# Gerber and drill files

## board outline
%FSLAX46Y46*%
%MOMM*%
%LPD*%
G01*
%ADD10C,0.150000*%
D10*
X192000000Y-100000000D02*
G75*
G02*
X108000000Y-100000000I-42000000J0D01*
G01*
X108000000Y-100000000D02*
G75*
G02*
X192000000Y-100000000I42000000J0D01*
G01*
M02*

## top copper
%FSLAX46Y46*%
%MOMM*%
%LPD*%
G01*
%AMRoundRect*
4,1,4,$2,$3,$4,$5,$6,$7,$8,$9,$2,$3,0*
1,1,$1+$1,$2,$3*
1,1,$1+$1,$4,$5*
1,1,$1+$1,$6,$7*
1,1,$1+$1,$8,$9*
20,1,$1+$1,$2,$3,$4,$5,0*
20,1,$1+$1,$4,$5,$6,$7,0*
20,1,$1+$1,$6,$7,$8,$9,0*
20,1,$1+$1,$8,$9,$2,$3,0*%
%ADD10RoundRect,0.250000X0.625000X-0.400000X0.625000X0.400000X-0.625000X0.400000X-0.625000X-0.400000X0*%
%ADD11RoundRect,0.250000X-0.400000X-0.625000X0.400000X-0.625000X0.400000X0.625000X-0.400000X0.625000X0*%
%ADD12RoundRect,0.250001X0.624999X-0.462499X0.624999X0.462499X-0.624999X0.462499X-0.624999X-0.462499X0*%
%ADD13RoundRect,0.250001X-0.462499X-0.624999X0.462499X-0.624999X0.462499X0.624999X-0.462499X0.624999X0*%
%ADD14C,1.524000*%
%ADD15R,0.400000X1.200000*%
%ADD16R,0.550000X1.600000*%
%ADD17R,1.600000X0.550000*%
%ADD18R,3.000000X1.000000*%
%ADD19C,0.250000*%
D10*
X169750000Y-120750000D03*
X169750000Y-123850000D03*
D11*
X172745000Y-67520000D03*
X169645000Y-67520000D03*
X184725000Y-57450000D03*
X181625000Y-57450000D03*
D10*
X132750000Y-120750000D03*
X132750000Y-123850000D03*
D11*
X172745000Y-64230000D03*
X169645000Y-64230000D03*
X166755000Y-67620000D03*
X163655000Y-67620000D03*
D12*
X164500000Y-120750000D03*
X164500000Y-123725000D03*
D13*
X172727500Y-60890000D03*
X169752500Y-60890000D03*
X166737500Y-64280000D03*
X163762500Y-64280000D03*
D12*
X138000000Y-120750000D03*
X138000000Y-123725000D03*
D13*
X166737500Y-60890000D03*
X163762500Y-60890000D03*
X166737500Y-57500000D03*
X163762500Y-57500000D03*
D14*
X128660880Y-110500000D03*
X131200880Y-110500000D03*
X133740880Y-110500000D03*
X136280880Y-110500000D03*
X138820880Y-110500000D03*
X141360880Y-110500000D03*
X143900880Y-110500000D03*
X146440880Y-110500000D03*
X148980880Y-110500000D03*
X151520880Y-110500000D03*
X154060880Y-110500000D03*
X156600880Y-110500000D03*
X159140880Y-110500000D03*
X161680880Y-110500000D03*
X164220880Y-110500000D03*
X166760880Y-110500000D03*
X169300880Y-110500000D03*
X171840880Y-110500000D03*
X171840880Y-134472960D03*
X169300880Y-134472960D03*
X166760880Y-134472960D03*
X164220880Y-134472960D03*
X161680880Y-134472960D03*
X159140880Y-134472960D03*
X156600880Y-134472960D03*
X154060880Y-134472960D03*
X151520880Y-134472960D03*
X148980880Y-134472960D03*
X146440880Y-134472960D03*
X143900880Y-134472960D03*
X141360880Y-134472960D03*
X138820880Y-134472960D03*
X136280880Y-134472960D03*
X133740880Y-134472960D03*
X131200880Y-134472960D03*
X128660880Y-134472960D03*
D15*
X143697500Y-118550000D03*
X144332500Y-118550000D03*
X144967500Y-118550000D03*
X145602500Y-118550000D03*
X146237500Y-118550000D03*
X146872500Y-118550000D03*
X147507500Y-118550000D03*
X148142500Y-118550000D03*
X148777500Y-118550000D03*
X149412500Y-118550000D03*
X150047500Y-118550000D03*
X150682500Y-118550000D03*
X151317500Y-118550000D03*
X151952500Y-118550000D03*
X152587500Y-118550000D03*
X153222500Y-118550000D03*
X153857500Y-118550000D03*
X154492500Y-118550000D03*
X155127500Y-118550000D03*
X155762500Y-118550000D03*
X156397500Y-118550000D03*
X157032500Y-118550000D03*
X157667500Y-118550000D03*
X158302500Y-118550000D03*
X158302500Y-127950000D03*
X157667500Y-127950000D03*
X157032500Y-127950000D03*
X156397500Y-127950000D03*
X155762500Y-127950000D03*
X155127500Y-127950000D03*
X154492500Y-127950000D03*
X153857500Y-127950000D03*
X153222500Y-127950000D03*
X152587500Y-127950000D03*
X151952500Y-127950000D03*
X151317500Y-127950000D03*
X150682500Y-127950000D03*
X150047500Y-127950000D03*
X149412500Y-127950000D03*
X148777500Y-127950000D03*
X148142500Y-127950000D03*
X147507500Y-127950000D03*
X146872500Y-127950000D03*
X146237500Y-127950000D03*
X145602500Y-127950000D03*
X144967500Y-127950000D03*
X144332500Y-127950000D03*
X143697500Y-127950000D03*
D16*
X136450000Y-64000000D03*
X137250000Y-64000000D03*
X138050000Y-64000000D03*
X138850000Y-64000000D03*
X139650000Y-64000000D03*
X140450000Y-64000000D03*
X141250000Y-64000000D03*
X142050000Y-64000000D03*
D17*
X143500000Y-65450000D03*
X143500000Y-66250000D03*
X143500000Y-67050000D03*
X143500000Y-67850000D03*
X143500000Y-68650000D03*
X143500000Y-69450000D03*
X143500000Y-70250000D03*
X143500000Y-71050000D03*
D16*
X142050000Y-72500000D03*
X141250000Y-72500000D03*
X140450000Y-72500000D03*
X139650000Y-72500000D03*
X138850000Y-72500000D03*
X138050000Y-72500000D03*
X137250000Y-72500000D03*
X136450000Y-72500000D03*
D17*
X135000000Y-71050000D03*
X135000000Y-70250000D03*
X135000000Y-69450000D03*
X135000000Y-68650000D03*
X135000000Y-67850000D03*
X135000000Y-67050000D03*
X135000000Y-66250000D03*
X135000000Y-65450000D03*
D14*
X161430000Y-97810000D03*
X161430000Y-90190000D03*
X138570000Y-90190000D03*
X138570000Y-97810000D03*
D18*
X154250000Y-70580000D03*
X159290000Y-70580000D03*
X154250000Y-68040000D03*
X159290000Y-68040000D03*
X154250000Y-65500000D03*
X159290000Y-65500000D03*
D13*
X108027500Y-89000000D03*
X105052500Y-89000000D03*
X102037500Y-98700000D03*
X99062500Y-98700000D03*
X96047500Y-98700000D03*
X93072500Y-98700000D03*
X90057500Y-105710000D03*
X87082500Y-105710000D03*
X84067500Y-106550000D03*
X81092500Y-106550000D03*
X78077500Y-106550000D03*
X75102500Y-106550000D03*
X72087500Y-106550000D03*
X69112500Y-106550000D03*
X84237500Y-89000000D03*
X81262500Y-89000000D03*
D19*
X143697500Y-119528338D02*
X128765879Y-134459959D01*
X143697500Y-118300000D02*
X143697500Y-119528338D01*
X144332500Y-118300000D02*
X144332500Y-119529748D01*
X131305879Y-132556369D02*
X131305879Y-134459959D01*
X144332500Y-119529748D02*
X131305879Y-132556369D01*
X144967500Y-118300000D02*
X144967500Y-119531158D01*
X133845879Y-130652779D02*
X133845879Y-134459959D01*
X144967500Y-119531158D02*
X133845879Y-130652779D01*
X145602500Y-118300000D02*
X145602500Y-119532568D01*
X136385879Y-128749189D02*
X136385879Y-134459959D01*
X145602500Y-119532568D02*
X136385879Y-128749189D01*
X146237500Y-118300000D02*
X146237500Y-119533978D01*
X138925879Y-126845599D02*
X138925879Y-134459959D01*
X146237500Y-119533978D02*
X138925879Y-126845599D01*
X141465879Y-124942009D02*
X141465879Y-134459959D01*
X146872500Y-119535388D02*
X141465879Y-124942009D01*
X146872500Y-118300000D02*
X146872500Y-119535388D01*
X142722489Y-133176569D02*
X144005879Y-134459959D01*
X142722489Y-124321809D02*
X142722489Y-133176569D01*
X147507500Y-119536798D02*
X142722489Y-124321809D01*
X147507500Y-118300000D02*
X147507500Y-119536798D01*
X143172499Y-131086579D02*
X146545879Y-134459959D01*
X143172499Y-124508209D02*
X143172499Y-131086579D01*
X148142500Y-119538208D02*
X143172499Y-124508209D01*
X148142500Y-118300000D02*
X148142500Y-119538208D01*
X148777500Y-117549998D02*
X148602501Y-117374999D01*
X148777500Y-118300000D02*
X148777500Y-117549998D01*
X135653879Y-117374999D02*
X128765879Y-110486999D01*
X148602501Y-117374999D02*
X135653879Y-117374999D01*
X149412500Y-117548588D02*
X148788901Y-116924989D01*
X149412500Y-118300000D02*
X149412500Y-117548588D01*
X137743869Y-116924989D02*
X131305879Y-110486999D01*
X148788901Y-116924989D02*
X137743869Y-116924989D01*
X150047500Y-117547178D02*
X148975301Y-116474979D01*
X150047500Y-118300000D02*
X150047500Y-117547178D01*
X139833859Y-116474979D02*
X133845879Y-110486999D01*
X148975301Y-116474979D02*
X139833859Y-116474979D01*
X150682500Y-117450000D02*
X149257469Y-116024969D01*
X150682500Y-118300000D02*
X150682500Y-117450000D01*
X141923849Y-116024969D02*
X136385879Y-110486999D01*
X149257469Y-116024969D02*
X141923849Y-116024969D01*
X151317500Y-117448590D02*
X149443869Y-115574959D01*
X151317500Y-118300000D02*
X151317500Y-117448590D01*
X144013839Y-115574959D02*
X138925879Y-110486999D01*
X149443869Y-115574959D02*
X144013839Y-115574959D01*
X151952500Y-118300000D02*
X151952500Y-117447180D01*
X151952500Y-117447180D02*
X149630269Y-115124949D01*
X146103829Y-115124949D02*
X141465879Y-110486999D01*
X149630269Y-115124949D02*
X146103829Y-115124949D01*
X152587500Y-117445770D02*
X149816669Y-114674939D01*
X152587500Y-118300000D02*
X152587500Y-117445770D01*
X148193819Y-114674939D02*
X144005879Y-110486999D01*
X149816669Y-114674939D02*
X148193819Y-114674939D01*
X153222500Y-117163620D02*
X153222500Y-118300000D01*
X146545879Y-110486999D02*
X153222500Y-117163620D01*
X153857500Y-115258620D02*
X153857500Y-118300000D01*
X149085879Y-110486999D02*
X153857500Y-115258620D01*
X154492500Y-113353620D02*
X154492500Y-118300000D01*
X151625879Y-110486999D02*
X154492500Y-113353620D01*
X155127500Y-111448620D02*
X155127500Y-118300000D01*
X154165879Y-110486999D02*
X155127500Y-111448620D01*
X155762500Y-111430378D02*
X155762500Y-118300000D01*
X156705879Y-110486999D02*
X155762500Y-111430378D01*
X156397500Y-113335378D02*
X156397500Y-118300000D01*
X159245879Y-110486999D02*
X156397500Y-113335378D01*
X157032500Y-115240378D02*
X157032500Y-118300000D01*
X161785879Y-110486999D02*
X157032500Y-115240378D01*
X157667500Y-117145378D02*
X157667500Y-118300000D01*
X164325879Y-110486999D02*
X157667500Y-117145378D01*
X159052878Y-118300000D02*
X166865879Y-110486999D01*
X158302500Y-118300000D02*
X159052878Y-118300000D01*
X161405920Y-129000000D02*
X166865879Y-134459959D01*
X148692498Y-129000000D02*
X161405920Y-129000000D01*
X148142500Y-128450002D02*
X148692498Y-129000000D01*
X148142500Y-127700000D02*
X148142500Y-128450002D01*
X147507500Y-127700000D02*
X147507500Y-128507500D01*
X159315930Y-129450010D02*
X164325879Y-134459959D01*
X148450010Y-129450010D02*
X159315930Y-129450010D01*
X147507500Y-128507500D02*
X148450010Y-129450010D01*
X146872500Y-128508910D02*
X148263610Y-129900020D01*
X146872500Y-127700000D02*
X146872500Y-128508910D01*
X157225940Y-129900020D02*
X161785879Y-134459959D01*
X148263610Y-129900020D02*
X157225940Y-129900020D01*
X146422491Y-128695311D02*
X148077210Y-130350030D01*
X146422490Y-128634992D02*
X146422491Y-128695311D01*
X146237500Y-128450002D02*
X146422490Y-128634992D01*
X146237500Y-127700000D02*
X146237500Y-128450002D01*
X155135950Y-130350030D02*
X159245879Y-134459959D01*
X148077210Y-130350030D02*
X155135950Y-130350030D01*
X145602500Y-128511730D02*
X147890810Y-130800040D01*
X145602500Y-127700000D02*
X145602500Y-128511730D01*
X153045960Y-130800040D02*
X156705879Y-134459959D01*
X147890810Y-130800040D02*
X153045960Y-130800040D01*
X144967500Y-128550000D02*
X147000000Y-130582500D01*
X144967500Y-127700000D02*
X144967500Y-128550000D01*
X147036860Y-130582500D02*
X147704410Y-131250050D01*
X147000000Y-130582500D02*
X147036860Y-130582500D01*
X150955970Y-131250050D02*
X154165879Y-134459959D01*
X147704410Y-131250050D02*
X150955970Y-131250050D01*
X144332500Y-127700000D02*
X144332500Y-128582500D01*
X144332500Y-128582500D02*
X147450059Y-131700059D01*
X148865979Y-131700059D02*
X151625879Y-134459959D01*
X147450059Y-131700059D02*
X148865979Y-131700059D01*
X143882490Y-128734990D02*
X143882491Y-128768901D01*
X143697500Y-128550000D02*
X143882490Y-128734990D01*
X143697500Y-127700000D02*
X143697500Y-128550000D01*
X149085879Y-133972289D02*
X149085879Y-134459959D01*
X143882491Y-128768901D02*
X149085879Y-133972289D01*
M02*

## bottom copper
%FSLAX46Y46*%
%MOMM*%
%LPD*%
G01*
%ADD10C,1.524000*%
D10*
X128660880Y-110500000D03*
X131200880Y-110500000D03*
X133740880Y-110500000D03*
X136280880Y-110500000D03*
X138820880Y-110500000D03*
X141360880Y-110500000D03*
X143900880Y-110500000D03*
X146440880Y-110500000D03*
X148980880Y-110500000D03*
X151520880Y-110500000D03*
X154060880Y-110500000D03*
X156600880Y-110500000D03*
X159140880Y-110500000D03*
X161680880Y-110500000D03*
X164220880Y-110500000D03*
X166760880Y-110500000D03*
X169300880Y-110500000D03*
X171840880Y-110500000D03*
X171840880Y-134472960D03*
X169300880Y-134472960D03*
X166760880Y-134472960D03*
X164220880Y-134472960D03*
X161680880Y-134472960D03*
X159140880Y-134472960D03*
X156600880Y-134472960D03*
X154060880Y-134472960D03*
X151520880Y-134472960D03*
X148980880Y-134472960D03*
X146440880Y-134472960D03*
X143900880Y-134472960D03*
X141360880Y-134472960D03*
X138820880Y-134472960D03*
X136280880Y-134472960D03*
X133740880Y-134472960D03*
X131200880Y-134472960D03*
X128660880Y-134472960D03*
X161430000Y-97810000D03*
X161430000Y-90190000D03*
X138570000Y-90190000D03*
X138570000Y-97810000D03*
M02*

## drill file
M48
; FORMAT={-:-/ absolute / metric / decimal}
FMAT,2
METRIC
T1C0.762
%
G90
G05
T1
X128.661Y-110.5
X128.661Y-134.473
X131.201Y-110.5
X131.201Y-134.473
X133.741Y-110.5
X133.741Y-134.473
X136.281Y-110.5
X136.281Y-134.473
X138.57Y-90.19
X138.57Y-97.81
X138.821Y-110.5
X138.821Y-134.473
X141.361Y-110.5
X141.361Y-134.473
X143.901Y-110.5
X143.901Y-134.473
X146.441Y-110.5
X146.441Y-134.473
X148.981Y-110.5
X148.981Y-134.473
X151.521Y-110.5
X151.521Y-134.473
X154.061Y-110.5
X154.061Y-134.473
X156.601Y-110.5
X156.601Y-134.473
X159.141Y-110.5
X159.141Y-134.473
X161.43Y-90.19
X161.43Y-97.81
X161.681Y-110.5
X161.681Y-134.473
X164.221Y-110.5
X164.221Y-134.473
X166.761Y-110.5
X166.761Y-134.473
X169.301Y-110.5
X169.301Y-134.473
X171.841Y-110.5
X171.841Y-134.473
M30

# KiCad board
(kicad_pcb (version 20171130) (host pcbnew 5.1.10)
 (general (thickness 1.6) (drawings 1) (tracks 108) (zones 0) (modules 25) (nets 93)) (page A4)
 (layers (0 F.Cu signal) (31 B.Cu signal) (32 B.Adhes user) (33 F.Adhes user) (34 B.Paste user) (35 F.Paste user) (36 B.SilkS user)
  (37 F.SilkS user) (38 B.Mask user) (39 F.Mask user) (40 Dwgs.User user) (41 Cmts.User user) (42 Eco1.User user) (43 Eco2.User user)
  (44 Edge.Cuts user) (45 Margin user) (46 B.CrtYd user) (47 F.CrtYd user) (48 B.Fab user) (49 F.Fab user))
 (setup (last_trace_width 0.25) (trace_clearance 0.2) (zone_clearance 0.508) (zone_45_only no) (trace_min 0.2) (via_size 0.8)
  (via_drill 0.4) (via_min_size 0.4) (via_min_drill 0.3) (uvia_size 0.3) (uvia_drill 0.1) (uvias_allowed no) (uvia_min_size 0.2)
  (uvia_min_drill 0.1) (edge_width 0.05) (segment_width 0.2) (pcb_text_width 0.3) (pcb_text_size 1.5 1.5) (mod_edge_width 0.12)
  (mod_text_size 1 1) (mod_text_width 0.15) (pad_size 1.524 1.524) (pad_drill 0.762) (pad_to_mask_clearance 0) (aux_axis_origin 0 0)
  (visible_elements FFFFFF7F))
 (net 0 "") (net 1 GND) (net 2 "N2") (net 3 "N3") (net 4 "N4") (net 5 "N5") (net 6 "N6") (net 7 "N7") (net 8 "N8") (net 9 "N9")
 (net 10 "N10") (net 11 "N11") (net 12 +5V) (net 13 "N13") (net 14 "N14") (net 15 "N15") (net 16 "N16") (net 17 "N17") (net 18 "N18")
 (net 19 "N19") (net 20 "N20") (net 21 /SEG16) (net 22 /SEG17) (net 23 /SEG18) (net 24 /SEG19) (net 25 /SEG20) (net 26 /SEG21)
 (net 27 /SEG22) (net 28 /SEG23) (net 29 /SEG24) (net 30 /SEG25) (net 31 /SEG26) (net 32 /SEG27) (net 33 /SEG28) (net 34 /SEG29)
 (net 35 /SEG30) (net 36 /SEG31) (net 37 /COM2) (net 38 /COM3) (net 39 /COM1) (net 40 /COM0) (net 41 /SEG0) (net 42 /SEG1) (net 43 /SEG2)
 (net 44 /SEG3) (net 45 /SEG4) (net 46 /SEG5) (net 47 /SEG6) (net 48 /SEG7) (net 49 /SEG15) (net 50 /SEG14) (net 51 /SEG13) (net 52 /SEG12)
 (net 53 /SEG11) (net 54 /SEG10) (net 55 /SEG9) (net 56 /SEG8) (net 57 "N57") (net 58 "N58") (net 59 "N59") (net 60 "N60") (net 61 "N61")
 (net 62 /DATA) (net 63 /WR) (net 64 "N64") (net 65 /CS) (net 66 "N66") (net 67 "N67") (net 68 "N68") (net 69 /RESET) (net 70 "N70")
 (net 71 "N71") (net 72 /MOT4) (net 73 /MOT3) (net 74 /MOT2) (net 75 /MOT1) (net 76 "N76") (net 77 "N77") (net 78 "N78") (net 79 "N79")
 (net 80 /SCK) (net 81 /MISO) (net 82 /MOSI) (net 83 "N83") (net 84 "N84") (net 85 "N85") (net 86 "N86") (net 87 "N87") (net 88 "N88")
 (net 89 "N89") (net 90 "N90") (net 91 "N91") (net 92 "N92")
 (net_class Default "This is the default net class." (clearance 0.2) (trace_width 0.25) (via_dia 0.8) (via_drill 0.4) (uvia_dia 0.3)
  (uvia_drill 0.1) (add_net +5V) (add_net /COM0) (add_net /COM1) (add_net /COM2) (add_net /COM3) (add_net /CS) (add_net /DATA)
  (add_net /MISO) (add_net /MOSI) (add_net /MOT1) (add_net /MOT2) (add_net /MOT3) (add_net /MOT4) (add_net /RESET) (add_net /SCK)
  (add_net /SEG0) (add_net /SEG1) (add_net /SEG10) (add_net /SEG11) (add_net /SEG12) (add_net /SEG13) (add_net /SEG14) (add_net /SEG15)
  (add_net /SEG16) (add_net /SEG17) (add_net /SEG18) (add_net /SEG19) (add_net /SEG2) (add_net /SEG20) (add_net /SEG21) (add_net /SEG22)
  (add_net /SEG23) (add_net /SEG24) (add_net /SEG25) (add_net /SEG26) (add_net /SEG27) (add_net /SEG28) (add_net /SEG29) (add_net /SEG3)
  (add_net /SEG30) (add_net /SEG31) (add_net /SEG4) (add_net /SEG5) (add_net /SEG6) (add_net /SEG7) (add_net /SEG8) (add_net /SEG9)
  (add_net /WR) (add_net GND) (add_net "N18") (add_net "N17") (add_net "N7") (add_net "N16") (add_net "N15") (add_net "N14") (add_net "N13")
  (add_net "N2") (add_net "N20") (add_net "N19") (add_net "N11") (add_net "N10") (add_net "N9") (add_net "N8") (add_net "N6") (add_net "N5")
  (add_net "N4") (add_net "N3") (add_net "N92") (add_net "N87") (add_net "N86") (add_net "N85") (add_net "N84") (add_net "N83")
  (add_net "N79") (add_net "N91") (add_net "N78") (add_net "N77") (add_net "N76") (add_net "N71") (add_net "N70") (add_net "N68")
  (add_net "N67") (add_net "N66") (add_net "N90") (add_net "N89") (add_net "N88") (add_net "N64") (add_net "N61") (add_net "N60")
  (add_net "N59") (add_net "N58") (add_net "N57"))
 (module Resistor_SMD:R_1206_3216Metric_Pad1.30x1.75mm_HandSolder (layer F.Cu) (at 169.75 122.3 90)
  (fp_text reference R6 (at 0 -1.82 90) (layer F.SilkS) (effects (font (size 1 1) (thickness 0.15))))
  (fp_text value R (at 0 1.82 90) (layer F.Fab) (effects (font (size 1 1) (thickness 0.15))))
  (pad 2 smd roundrect (at 1.55 0 90) (size 1.3 1.75) (layers F.Cu F.Paste F.Mask) (roundrect_rratio 0.192308) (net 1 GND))
  (pad 1 smd roundrect (at -1.55 0 90) (size 1.3 1.75) (layers F.Cu F.Paste F.Mask) (roundrect_rratio 0.192308) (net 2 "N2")))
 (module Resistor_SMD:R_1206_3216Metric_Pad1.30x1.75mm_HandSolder (layer F.Cu) (at 171.195 67.52)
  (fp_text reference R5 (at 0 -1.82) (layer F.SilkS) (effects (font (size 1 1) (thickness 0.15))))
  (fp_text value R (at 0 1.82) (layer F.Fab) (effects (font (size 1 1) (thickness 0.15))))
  (pad 2 smd roundrect (at 1.55 0) (size 1.3 1.75) (layers F.Cu F.Paste F.Mask) (roundrect_rratio 0.192308) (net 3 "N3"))
  (pad 1 smd roundrect (at -1.55 0) (size 1.3 1.75) (layers F.Cu F.Paste F.Mask) (roundrect_rratio 0.192308) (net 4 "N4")))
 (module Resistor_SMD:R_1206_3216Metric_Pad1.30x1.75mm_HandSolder (layer F.Cu) (at 183.175 57.45)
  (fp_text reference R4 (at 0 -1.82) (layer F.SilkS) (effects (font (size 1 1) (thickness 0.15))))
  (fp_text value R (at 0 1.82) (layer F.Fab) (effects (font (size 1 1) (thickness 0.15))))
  (pad 2 smd roundrect (at 1.55 0) (size 1.3 1.75) (layers F.Cu F.Paste F.Mask) (roundrect_rratio 0.192308) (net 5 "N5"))
  (pad 1 smd roundrect (at -1.55 0) (size 1.3 1.75) (layers F.Cu F.Paste F.Mask) (roundrect_rratio 0.192308) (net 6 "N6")))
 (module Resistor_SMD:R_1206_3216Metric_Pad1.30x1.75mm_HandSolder (layer F.Cu) (at 132.75 122.3 90)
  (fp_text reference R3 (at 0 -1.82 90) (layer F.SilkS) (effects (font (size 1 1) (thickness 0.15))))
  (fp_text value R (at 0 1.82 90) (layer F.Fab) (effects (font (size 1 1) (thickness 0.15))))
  (pad 2 smd roundrect (at 1.55 0 90) (size 1.3 1.75) (layers F.Cu F.Paste F.Mask) (roundrect_rratio 0.192308) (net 1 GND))
  (pad 1 smd roundrect (at -1.55 0 90) (size 1.3 1.75) (layers F.Cu F.Paste F.Mask) (roundrect_rratio 0.192308) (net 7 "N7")))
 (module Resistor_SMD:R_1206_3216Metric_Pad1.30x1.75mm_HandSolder (layer F.Cu) (at 171.195 64.23)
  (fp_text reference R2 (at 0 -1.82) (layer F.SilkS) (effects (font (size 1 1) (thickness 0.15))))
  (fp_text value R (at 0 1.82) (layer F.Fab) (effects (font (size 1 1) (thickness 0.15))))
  (pad 2 smd roundrect (at 1.55 0) (size 1.3 1.75) (layers F.Cu F.Paste F.Mask) (roundrect_rratio 0.192308) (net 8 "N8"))
  (pad 1 smd roundrect (at -1.55 0) (size 1.3 1.75) (layers F.Cu F.Paste F.Mask) (roundrect_rratio 0.192308) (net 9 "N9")))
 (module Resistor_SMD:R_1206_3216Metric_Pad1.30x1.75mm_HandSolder (layer F.Cu) (at 165.205 67.62)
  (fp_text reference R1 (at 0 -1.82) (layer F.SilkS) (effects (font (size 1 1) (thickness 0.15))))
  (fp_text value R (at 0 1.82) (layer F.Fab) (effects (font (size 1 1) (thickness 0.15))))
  (pad 2 smd roundrect (at 1.55 0) (size 1.3 1.75) (layers F.Cu F.Paste F.Mask) (roundrect_rratio 0.192308) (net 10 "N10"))
  (pad 1 smd roundrect (at -1.55 0) (size 1.3 1.75) (layers F.Cu F.Paste F.Mask) (roundrect_rratio 0.192308) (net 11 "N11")))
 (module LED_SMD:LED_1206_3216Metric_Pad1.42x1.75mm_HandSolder (layer F.Cu) (at 164.5 122.2375 90)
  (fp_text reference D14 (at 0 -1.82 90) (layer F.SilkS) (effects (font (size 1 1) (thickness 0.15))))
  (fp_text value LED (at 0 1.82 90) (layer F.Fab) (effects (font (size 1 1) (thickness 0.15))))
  (pad 2 smd roundrect (at 1.4875 0 90) (size 1.425 1.75) (layers F.Cu F.Paste F.Mask) (roundrect_rratio 0.175439) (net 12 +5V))
  (pad 1 smd roundrect (at -1.4875 0 90) (size 1.425 1.75) (layers F.Cu F.Paste F.Mask) (roundrect_rratio 0.175439) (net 2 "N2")))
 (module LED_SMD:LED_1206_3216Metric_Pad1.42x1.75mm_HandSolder (layer F.Cu) (at 171.24 60.89)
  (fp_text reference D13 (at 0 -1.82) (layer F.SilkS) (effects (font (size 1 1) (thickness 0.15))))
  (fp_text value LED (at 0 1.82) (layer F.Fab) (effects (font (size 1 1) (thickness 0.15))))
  (pad 2 smd roundrect (at 1.4875 0) (size 1.425 1.75) (layers F.Cu F.Paste F.Mask) (roundrect_rratio 0.175439) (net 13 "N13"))
  (pad 1 smd roundrect (at -1.4875 0) (size 1.425 1.75) (layers F.Cu F.Paste F.Mask) (roundrect_rratio 0.175439) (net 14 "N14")))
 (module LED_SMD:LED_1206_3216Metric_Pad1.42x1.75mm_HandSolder (layer F.Cu) (at 165.25 64.28)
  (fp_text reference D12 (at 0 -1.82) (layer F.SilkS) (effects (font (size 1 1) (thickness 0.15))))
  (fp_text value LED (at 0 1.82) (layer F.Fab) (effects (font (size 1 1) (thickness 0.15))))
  (pad 2 smd roundrect (at 1.4875 0) (size 1.425 1.75) (layers F.Cu F.Paste F.Mask) (roundrect_rratio 0.175439) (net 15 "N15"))
  (pad 1 smd roundrect (at -1.4875 0) (size 1.425 1.75) (layers F.Cu F.Paste F.Mask) (roundrect_rratio 0.175439) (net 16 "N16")))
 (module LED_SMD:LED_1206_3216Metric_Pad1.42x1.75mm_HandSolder (layer F.Cu) (at 138 122.2375 90)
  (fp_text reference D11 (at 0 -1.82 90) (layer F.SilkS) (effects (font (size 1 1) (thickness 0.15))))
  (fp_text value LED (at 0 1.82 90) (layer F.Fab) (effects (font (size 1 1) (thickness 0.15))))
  (pad 2 smd roundrect (at 1.4875 0 90) (size 1.425 1.75) (layers F.Cu F.Paste F.Mask) (roundrect_rratio 0.175439) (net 12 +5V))
  (pad 1 smd roundrect (at -1.4875 0 90) (size 1.425 1.75) (layers F.Cu F.Paste F.Mask) (roundrect_rratio 0.175439) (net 7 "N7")))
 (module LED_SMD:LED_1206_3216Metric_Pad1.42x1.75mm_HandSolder (layer F.Cu) (at 165.25 60.89)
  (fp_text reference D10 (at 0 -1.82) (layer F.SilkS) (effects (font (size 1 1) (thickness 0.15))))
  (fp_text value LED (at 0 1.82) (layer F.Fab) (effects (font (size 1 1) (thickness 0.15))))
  (pad 2 smd roundrect (at 1.4875 0) (size 1.425 1.75) (layers F.Cu F.Paste F.Mask) (roundrect_rratio 0.175439) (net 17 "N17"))
  (pad 1 smd roundrect (at -1.4875 0) (size 1.425 1.75) (layers F.Cu F.Paste F.Mask) (roundrect_rratio 0.175439) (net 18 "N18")))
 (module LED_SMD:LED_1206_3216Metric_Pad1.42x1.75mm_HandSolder (layer F.Cu) (at 165.25 57.5)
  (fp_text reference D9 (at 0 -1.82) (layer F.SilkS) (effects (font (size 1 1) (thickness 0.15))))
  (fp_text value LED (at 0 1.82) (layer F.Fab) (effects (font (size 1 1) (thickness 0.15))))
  (pad 2 smd roundrect (at 1.4875 0) (size 1.425 1.75) (layers F.Cu F.Paste F.Mask) (roundrect_rratio 0.175439) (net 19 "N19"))
  (pad 1 smd roundrect (at -1.4875 0) (size 1.425 1.75) (layers F.Cu F.Paste F.Mask) (roundrect_rratio 0.175439) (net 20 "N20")))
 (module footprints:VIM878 (layer F.Cu) (at 124.25 112.97296)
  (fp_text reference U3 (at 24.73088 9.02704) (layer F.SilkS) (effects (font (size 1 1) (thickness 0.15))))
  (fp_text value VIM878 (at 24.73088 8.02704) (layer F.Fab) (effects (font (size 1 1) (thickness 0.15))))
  (pad 36 thru_hole circle (at 4.41088 -2.47296) (size 1.524 1.524) (drill 0.762) (layers *.Cu *.Mask) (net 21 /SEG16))
  (pad 35 thru_hole circle (at 6.95088 -2.47296) (size 1.524 1.524) (drill 0.762) (layers *.Cu *.Mask) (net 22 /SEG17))
  (pad 34 thru_hole circle (at 9.49088 -2.47296) (size 1.524 1.524) (drill 0.762) (layers *.Cu *.Mask) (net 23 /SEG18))
  (pad 33 thru_hole circle (at 12.03088 -2.47296) (size 1.524 1.524) (drill 0.762) (layers *.Cu *.Mask) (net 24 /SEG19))
  (pad 32 thru_hole circle (at 14.57088 -2.47296) (size 1.524 1.524) (drill 0.762) (layers *.Cu *.Mask) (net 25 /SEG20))
  (pad 31 thru_hole circle (at 17.11088 -2.47296) (size 1.524 1.524) (drill 0.762) (layers *.Cu *.Mask) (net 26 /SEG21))
  (pad 30 thru_hole circle (at 19.65088 -2.47296) (size 1.524 1.524) (drill 0.762) (layers *.Cu *.Mask) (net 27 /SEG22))
  (pad 29 thru_hole circle (at 22.19088 -2.47296) (size 1.524 1.524) (drill 0.762) (layers *.Cu *.Mask) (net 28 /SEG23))
  (pad 28 thru_hole circle (at 24.73088 -2.47296) (size 1.524 1.524) (drill 0.762) (layers *.Cu *.Mask) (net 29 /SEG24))
  (pad 27 thru_hole circle (at 27.27088 -2.47296) (size 1.524 1.524) (drill 0.762) (layers *.Cu *.Mask) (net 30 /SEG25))
  (pad 26 thru_hole circle (at 29.81088 -2.47296) (size 1.524 1.524) (drill 0.762) (layers *.Cu *.Mask) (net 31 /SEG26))
  (pad 25 thru_hole circle (at 32.35088 -2.47296) (size 1.524 1.524) (drill 0.762) (layers *.Cu *.Mask) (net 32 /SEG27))
  (pad 24 thru_hole circle (at 34.89088 -2.47296) (size 1.524 1.524) (drill 0.762) (layers *.Cu *.Mask) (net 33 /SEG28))
  (pad 23 thru_hole circle (at 37.43088 -2.47296) (size 1.524 1.524) (drill 0.762) (layers *.Cu *.Mask) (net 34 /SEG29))
  (pad 22 thru_hole circle (at 39.97088 -2.47296) (size 1.524 1.524) (drill 0.762) (layers *.Cu *.Mask) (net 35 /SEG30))
  (pad 21 thru_hole circle (at 42.51088 -2.47296) (size 1.524 1.524) (drill 0.762) (layers *.Cu *.Mask) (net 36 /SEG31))
  (pad 20 thru_hole circle (at 45.05088 -2.47296) (size 1.524 1.524) (drill 0.762) (layers *.Cu *.Mask) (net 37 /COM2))
  (pad 19 thru_hole circle (at 47.59088 -2.47296) (size 1.524 1.524) (drill 0.762) (layers *.Cu *.Mask) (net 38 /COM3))
  (pad 18 thru_hole circle (at 47.59088 21.5) (size 1.524 1.524) (drill 0.762) (layers *.Cu *.Mask) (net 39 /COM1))
  (pad 17 thru_hole circle (at 45.05088 21.5) (size 1.524 1.524) (drill 0.762) (layers *.Cu *.Mask) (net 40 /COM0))
  (pad 16 thru_hole circle (at 42.51088 21.5) (size 1.524 1.524) (drill 0.762) (layers *.Cu *.Mask) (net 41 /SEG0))
  (pad 15 thru_hole circle (at 39.97088 21.5) (size 1.524 1.524) (drill 0.762) (layers *.Cu *.Mask) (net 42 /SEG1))
  (pad 14 thru_hole circle (at 37.43088 21.5) (size 1.524 1.524) (drill 0.762) (layers *.Cu *.Mask) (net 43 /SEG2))
  (pad 13 thru_hole circle (at 34.89088 21.5) (size 1.524 1.524) (drill 0.762) (layers *.Cu *.Mask) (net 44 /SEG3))
  (pad 12 thru_hole circle (at 32.35088 21.5) (size 1.524 1.524) (drill 0.762) (layers *.Cu *.Mask) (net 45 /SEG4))
  (pad 11 thru_hole circle (at 29.81088 21.5) (size 1.524 1.524) (drill 0.762) (layers *.Cu *.Mask) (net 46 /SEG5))
  (pad 10 thru_hole circle (at 27.27088 21.5) (size 1.524 1.524) (drill 0.762) (layers *.Cu *.Mask) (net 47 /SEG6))
  (pad 9 thru_hole circle (at 24.73088 21.5) (size 1.524 1.524) (drill 0.762) (layers *.Cu *.Mask) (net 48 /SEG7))
  (pad 8 thru_hole circle (at 22.19088 21.5) (size 1.524 1.524) (drill 0.762) (layers *.Cu *.Mask) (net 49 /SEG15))
  (pad 7 thru_hole circle (at 19.65088 21.5) (size 1.524 1.524) (drill 0.762) (layers *.Cu *.Mask) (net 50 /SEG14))
  (pad 6 thru_hole circle (at 17.11088 21.5) (size 1.524 1.524) (drill 0.762) (layers *.Cu *.Mask) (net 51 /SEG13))
  (pad 5 thru_hole circle (at 14.57088 21.5) (size 1.524 1.524) (drill 0.762) (layers *.Cu *.Mask) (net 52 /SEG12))
  (pad 4 thru_hole circle (at 12.03088 21.5) (size 1.524 1.524) (drill 0.762) (layers *.Cu *.Mask) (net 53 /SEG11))
  (pad 3 thru_hole circle (at 9.49088 21.5) (size 1.524 1.524) (drill 0.762) (layers *.Cu *.Mask) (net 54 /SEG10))
  (pad 2 thru_hole circle (at 6.95088 21.5) (size 1.524 1.524) (drill 0.762) (layers *.Cu *.Mask) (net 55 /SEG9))
  (pad 1 thru_hole circle (at 4.41088 21.5) (size 1.524 1.524) (drill 0.762) (layers *.Cu *.Mask) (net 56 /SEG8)))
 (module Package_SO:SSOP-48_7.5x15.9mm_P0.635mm (layer F.Cu) (at 151 123.25 90)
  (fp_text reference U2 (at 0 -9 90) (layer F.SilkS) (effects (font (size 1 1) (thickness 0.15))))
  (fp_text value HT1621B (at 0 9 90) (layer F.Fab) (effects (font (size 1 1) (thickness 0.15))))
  (pad 48 smd rect (at 4.7 -7.3025 90) (size 1.2 0.4) (layers F.Cu F.Paste F.Mask) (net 56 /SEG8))
  (pad 47 smd rect (at 4.7 -6.6675 90) (size 1.2 0.4) (layers F.Cu F.Paste F.Mask) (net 55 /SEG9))
  (pad 46 smd rect (at 4.7 -6.0325 90) (size 1.2 0.4) (layers F.Cu F.Paste F.Mask) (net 54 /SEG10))
  (pad 45 smd rect (at 4.7 -5.3975 90) (size 1.2 0.4) (layers F.Cu F.Paste F.Mask) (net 53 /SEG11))
  (pad 44 smd rect (at 4.7 -4.7625 90) (size 1.2 0.4) (layers F.Cu F.Paste F.Mask) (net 52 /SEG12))
  (pad 43 smd rect (at 4.7 -4.1275 90) (size 1.2 0.4) (layers F.Cu F.Paste F.Mask) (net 51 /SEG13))
  (pad 42 smd rect (at 4.7 -3.4925 90) (size 1.2 0.4) (layers F.Cu F.Paste F.Mask) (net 50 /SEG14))
  (pad 41 smd rect (at 4.7 -2.8575 90) (size 1.2 0.4) (layers F.Cu F.Paste F.Mask) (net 49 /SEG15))
  (pad 40 smd rect (at 4.7 -2.2225 90) (size 1.2 0.4) (layers F.Cu F.Paste F.Mask) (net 21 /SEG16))
  (pad 39 smd rect (at 4.7 -1.5875 90) (size 1.2 0.4) (layers F.Cu F.Paste F.Mask) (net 22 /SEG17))
  (pad 38 smd rect (at 4.7 -0.9525 90) (size 1.2 0.4) (layers F.Cu F.Paste F.Mask) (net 23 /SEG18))
  (pad 37 smd rect (at 4.7 -0.3175 90) (size 1.2 0.4) (layers F.Cu F.Paste F.Mask) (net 24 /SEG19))
  (pad 36 smd rect (at 4.7 0.3175 90) (size 1.2 0.4) (layers F.Cu F.Paste F.Mask) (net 25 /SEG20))
  (pad 35 smd rect (at 4.7 0.9525 90) (size 1.2 0.4) (layers F.Cu F.Paste F.Mask) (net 26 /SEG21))
  (pad 34 smd rect (at 4.7 1.5875 90) (size 1.2 0.4) (layers F.Cu F.Paste F.Mask) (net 27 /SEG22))
  (pad 33 smd rect (at 4.7 2.2225 90) (size 1.2 0.4) (layers F.Cu F.Paste F.Mask) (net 28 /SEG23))
  (pad 32 smd rect (at 4.7 2.8575 90) (size 1.2 0.4) (layers F.Cu F.Paste F.Mask) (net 29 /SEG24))
  (pad 31 smd rect (at 4.7 3.4925 90) (size 1.2 0.4) (layers F.Cu F.Paste F.Mask) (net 30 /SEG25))
  (pad 30 smd rect (at 4.7 4.1275 90) (size 1.2 0.4) (layers F.Cu F.Paste F.Mask) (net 31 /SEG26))
  (pad 29 smd rect (at 4.7 4.7625 90) (size 1.2 0.4) (layers F.Cu F.Paste F.Mask) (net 32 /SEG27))
  (pad 28 smd rect (at 4.7 5.3975 90) (size 1.2 0.4) (layers F.Cu F.Paste F.Mask) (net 33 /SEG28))
  (pad 27 smd rect (at 4.7 6.0325 90) (size 1.2 0.4) (layers F.Cu F.Paste F.Mask) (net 34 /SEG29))
  (pad 26 smd rect (at 4.7 6.6675 90) (size 1.2 0.4) (layers F.Cu F.Paste F.Mask) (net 35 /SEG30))
  (pad 25 smd rect (at 4.7 7.3025 90) (size 1.2 0.4) (layers F.Cu F.Paste F.Mask) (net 36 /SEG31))
  (pad 24 smd rect (at -4.7 7.3025 90) (size 1.2 0.4) (layers F.Cu F.Paste F.Mask) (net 38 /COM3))
  (pad 23 smd rect (at -4.7 6.6675 90) (size 1.2 0.4) (layers F.Cu F.Paste F.Mask) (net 37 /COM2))
  (pad 22 smd rect (at -4.7 6.0325 90) (size 1.2 0.4) (layers F.Cu F.Paste F.Mask) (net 39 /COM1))
  (pad 21 smd rect (at -4.7 5.3975 90) (size 1.2 0.4) (layers F.Cu F.Paste F.Mask) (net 40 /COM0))
  (pad 20 smd rect (at -4.7 4.7625 90) (size 1.2 0.4) (layers F.Cu F.Paste F.Mask) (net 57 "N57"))
  (pad 19 smd rect (at -4.7 4.1275 90) (size 1.2 0.4) (layers F.Cu F.Paste F.Mask) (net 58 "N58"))
  (pad 18 smd rect (at -4.7 3.4925 90) (size 1.2 0.4) (layers F.Cu F.Paste F.Mask) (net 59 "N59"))
  (pad 17 smd rect (at -4.7 2.8575 90) (size 1.2 0.4) (layers F.Cu F.Paste F.Mask) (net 12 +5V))
  (pad 16 smd rect (at -4.7 2.2225 90) (size 1.2 0.4) (layers F.Cu F.Paste F.Mask) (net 12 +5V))
  (pad 15 smd rect (at -4.7 1.5875 90) (size 1.2 0.4) (layers F.Cu F.Paste F.Mask) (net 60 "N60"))
  (pad 14 smd rect (at -4.7 0.9525 90) (size 1.2 0.4) (layers F.Cu F.Paste F.Mask) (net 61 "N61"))
  (pad 13 smd rect (at -4.7 0.3175 90) (size 1.2 0.4) (layers F.Cu F.Paste F.Mask) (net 1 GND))
  (pad 12 smd rect (at -4.7 -0.3175 90) (size 1.2 0.4) (layers F.Cu F.Paste F.Mask) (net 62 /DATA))
  (pad 11 smd rect (at -4.7 -0.9525 90) (size 1.2 0.4) (layers F.Cu F.Paste F.Mask) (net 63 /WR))
  (pad 10 smd rect (at -4.7 -1.5875 90) (size 1.2 0.4) (layers F.Cu F.Paste F.Mask) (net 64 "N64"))
  (pad 9 smd rect (at -4.7 -2.2225 90) (size 1.2 0.4) (layers F.Cu F.Paste F.Mask) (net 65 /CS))
  (pad 8 smd rect (at -4.7 -2.8575 90) (size 1.2 0.4) (layers F.Cu F.Paste F.Mask) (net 41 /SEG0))
  (pad 7 smd rect (at -4.7 -3.4925 90) (size 1.2 0.4) (layers F.Cu F.Paste F.Mask) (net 42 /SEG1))
  (pad 6 smd rect (at -4.7 -4.1275 90) (size 1.2 0.4) (layers F.Cu F.Paste F.Mask) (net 43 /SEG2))
  (pad 5 smd rect (at -4.7 -4.7625 90) (size 1.2 0.4) (layers F.Cu F.Paste F.Mask) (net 44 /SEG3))
  (pad 4 smd rect (at -4.7 -5.3975 90) (size 1.2 0.4) (layers F.Cu F.Paste F.Mask) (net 45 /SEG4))
  (pad 3 smd rect (at -4.7 -6.0325 90) (size 1.2 0.4) (layers F.Cu F.Paste F.Mask) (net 46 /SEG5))
  (pad 2 smd rect (at -4.7 -6.6675 90) (size 1.2 0.4) (layers F.Cu F.Paste F.Mask) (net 47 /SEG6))
  (pad 1 smd rect (at -4.7 -7.3025 90) (size 1.2 0.4) (layers F.Cu F.Paste F.Mask) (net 48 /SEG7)))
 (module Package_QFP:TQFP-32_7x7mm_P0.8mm (layer F.Cu) (at 139.25 68.25)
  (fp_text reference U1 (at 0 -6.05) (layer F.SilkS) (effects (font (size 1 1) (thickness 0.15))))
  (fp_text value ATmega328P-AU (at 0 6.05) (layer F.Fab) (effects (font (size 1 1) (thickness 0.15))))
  (pad 32 smd rect (at -2.8 -4.25 90) (size 1.6 0.55) (layers F.Cu F.Paste F.Mask) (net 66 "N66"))
  (pad 31 smd rect (at -2 -4.25 90) (size 1.6 0.55) (layers F.Cu F.Paste F.Mask) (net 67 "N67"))
  (pad 30 smd rect (at -1.2 -4.25 90) (size 1.6 0.55) (layers F.Cu F.Paste F.Mask) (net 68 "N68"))
  (pad 29 smd rect (at -0.4 -4.25 90) (size 1.6 0.55) (layers F.Cu F.Paste F.Mask) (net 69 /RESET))
  (pad 28 smd rect (at 0.4 -4.25 90) (size 1.6 0.55) (layers F.Cu F.Paste F.Mask) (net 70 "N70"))
  (pad 27 smd rect (at 1.2 -4.25 90) (size 1.6 0.55) (layers F.Cu F.Paste F.Mask) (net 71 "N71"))
  (pad 26 smd rect (at 2 -4.25 90) (size 1.6 0.55) (layers F.Cu F.Paste F.Mask) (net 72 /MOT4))
  (pad 25 smd rect (at 2.8 -4.25 90) (size 1.6 0.55) (layers F.Cu F.Paste F.Mask) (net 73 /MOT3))
  (pad 24 smd rect (at 4.25 -2.8) (size 1.6 0.55) (layers F.Cu F.Paste F.Mask) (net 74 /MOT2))
  (pad 23 smd rect (at 4.25 -2) (size 1.6 0.55) (layers F.Cu F.Paste F.Mask) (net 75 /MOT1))
  (pad 22 smd rect (at 4.25 -1.2) (size 1.6 0.55) (layers F.Cu F.Paste F.Mask) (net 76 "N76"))
  (pad 21 smd rect (at 4.25 -0.4) (size 1.6 0.55) (layers F.Cu F.Paste F.Mask) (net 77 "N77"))
  (pad 20 smd rect (at 4.25 0.4) (size 1.6 0.55) (layers F.Cu F.Paste F.Mask) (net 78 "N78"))
  (pad 19 smd rect (at 4.25 1.2) (size 1.6 0.55) (layers F.Cu F.Paste F.Mask) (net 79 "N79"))
  (pad 18 smd rect (at 4.25 2) (size 1.6 0.55) (layers F.Cu F.Paste F.Mask) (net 12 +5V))
  (pad 17 smd rect (at 4.25 2.8) (size 1.6 0.55) (layers F.Cu F.Paste F.Mask) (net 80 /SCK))
  (pad 16 smd rect (at 2.8 4.25 90) (size 1.6 0.55) (layers F.Cu F.Paste F.Mask) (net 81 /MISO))
  (pad 15 smd rect (at 2 4.25 90) (size 1.6 0.55) (layers F.Cu F.Paste F.Mask) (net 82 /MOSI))
  (pad 14 smd rect (at 1.2 4.25 90) (size 1.6 0.55) (layers F.Cu F.Paste F.Mask) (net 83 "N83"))
  (pad 13 smd rect (at 0.4 4.25 90) (size 1.6 0.55) (layers F.Cu F.Paste F.Mask) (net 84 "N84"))
  (pad 12 smd rect (at -0.4 4.25 90) (size 1.6 0.55) (layers F.Cu F.Paste F.Mask) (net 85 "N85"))
  (pad 11 smd rect (at -1.2 4.25 90) (size 1.6 0.55) (layers F.Cu F.Paste F.Mask) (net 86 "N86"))
  (pad 10 smd rect (at -2 4.25 90) (size 1.6 0.55) (layers F.Cu F.Paste F.Mask) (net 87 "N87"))
  (pad 9 smd rect (at -2.8 4.25 90) (size 1.6 0.55) (layers F.Cu F.Paste F.Mask) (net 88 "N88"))
  (pad 8 smd rect (at -4.25 2.8) (size 1.6 0.55) (layers F.Cu F.Paste F.Mask) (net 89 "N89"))
  (pad 7 smd rect (at -4.25 2) (size 1.6 0.55) (layers F.Cu F.Paste F.Mask) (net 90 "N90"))
  (pad 6 smd rect (at -4.25 1.2) (size 1.6 0.55) (layers F.Cu F.Paste F.Mask) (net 12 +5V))
  (pad 5 smd rect (at -4.25 0.4) (size 1.6 0.55) (layers F.Cu F.Paste F.Mask) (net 77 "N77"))
  (pad 4 smd rect (at -4.25 -0.4) (size 1.6 0.55) (layers F.Cu F.Paste F.Mask) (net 12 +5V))
  (pad 3 smd rect (at -4.25 -1.2) (size 1.6 0.55) (layers F.Cu F.Paste F.Mask) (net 77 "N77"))
  (pad 2 smd rect (at -4.25 -2) (size 1.6 0.55) (layers F.Cu F.Paste F.Mask) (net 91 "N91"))
  (pad 1 smd rect (at -4.25 -2.8) (size 1.6 0.55) (layers F.Cu F.Paste F.Mask) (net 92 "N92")))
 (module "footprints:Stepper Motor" (layer F.Cu) (at 150 94)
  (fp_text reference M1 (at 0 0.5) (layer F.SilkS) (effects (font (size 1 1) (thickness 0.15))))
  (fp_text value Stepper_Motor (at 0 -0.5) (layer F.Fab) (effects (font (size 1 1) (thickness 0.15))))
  (pad 4 thru_hole circle (at 11.43 3.81) (size 1.524 1.524) (drill 0.762) (layers *.Cu *.Mask) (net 72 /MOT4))
  (pad 3 thru_hole circle (at 11.43 -3.81) (size 1.524 1.524) (drill 0.762) (layers *.Cu *.Mask) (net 73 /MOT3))
  (pad 2 thru_hole circle (at -11.43 -3.81) (size 1.524 1.524) (drill 0.762) (layers *.Cu *.Mask) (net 74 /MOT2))
  (pad 1 thru_hole circle (at -11.43 3.81) (size 1.524 1.524) (drill 0.762) (layers *.Cu *.Mask) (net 75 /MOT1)))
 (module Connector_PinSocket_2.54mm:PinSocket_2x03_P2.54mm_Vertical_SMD (layer F.Cu) (at 156.77 68.04)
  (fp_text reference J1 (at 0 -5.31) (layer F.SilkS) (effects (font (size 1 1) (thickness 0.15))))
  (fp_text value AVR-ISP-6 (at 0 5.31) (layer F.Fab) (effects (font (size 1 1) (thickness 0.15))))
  (pad 6 smd rect (at -2.52 2.54) (size 3 1) (layers F.Cu F.Paste F.Mask) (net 1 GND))
  (pad 5 smd rect (at 2.52 2.54) (size 3 1) (layers F.Cu F.Paste F.Mask) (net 69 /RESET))
  (pad 4 smd rect (at -2.52 0) (size 3 1) (layers F.Cu F.Paste F.Mask) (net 82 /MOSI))
  (pad 3 smd rect (at 2.52 0) (size 3 1) (layers F.Cu F.Paste F.Mask) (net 80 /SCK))
  (pad 2 smd rect (at -2.52 -2.54) (size 3 1) (layers F.Cu F.Paste F.Mask) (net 12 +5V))
  (pad 1 smd rect (at 2.52 -2.54) (size 3 1) (layers F.Cu F.Paste F.Mask) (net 81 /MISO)))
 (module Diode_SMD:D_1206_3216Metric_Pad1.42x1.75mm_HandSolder (layer F.Cu) (at 106.54 89)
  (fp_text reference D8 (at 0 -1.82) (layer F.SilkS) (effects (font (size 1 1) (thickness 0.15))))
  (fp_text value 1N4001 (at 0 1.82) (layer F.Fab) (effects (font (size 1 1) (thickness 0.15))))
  (pad 2 smd roundrect (at 1.4875 0) (size 1.425 1.75) (layers F.Cu F.Paste F.Mask) (roundrect_rratio 0.175439) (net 1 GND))
  (pad 1 smd roundrect (at -1.4875 0) (size 1.425 1.75) (layers F.Cu F.Paste F.Mask) (roundrect_rratio 0.175439) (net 75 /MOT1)))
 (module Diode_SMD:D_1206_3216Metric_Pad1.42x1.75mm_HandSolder (layer F.Cu) (at 100.55 98.7)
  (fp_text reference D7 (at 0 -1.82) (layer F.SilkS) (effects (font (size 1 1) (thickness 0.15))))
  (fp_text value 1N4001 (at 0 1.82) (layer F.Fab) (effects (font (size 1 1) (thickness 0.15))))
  (pad 2 smd roundrect (at 1.4875 0) (size 1.425 1.75) (layers F.Cu F.Paste F.Mask) (roundrect_rratio 0.175439) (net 75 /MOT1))
  (pad 1 smd roundrect (at -1.4875 0) (size 1.425 1.75) (layers F.Cu F.Paste F.Mask) (roundrect_rratio 0.175439) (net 12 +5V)))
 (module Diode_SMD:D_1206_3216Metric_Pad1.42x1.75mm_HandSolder (layer F.Cu) (at 94.56 98.7)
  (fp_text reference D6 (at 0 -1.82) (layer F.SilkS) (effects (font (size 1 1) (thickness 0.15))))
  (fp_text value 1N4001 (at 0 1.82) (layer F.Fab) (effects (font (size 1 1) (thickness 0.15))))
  (pad 2 smd roundrect (at 1.4875 0) (size 1.425 1.75) (layers F.Cu F.Paste F.Mask) (roundrect_rratio 0.175439) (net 1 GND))
  (pad 1 smd roundrect (at -1.4875 0) (size 1.425 1.75) (layers F.Cu F.Paste F.Mask) (roundrect_rratio 0.175439) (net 74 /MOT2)))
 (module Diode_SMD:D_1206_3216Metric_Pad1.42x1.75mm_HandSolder (layer F.Cu) (at 88.57 105.71)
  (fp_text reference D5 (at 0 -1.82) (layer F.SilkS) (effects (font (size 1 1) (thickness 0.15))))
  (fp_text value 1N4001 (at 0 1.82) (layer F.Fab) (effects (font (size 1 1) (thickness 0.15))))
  (pad 2 smd roundrect (at 1.4875 0) (size 1.425 1.75) (layers F.Cu F.Paste F.Mask) (roundrect_rratio 0.175439) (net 74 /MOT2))
  (pad 1 smd roundrect (at -1.4875 0) (size 1.425 1.75) (layers F.Cu F.Paste F.Mask) (roundrect_rratio 0.175439) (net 12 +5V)))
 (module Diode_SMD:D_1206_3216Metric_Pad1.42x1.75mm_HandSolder (layer F.Cu) (at 82.58 106.55)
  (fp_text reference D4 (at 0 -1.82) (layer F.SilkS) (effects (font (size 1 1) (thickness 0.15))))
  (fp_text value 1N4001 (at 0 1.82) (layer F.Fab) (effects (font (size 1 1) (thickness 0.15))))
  (pad 2 smd roundrect (at 1.4875 0) (size 1.425 1.75) (layers F.Cu F.Paste F.Mask) (roundrect_rratio 0.175439) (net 1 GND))
  (pad 1 smd roundrect (at -1.4875 0) (size 1.425 1.75) (layers F.Cu F.Paste F.Mask) (roundrect_rratio 0.175439) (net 72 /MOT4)))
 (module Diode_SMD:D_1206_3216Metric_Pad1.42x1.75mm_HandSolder (layer F.Cu) (at 76.59 106.55)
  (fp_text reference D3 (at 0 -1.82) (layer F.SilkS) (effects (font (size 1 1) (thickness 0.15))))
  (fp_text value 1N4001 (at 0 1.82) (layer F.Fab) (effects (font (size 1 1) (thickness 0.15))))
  (pad 2 smd roundrect (at 1.4875 0) (size 1.425 1.75) (layers F.Cu F.Paste F.Mask) (roundrect_rratio 0.175439) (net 72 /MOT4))
  (pad 1 smd roundrect (at -1.4875 0) (size 1.425 1.75) (layers F.Cu F.Paste F.Mask) (roundrect_rratio 0.175439) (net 12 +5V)))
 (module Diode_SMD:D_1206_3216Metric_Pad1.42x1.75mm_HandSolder (layer F.Cu) (at 70.6 106.55)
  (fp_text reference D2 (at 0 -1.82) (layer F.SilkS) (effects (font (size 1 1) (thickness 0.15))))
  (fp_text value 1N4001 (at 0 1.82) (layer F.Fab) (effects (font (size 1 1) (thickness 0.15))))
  (pad 2 smd roundrect (at 1.4875 0) (size 1.425 1.75) (layers F.Cu F.Paste F.Mask) (roundrect_rratio 0.175439) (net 1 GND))
  (pad 1 smd roundrect (at -1.4875 0) (size 1.425 1.75) (layers F.Cu F.Paste F.Mask) (roundrect_rratio 0.175439) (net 73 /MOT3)))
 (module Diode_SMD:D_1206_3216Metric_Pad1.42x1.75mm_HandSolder (layer F.Cu) (at 82.75 89)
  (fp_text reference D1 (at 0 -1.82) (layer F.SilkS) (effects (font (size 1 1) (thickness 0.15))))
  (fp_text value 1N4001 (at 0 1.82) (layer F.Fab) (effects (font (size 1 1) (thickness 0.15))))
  (pad 2 smd roundrect (at 1.4875 0) (size 1.425 1.75) (layers F.Cu F.Paste F.Mask) (roundrect_rratio 0.175439) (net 73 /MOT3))
  (pad 1 smd roundrect (at -1.4875 0) (size 1.425 1.75) (layers F.Cu F.Paste F.Mask) (roundrect_rratio 0.175439) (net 12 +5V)))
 (gr_circle (center 150 100) (end 192 100) (layer Edge.Cuts) (width 0.15))
 (segment (start 143.6975 119.528338) (end 128.765879 134.459959) (width 0.25) (layer F.Cu) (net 56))
 (segment (start 143.6975 118.3) (end 143.6975 119.528338) (width 0.25) (layer F.Cu) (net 56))
 (segment (start 144.3325 118.3) (end 144.3325 119.529748) (width 0.25) (layer F.Cu) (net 55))
 (segment (start 131.305879 132.556369) (end 131.305879 134.459959) (width 0.25) (layer F.Cu) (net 55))
 (segment (start 144.3325 119.529748) (end 131.305879 132.556369) (width 0.25) (layer F.Cu) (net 55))
 (segment (start 144.9675 118.3) (end 144.9675 119.531158) (width 0.25) (layer F.Cu) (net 54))
 (segment (start 133.845879 130.652779) (end 133.845879 134.459959) (width 0.25) (layer F.Cu) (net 54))
 (segment (start 144.9675 119.531158) (end 133.845879 130.652779) (width 0.25) (layer F.Cu) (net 54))
 (segment (start 145.6025 118.3) (end 145.6025 119.532568) (width 0.25) (layer F.Cu) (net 53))
 (segment (start 136.385879 128.749189) (end 136.385879 134.459959) (width 0.25) (layer F.Cu) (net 53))
 (segment (start 145.6025 119.532568) (end 136.385879 128.749189) (width 0.25) (layer F.Cu) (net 53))
 (segment (start 146.2375 118.3) (end 146.2375 119.533978) (width 0.25) (layer F.Cu) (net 52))
 (segment (start 138.925879 126.845599) (end 138.925879 134.459959) (width 0.25) (layer F.Cu) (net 52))
 (segment (start 146.2375 119.533978) (end 138.925879 126.845599) (width 0.25) (layer F.Cu) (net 52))
 (segment (start 141.465879 124.942009) (end 141.465879 134.459959) (width 0.25) (layer F.Cu) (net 51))
 (segment (start 146.8725 119.535388) (end 141.465879 124.942009) (width 0.25) (layer F.Cu) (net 51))
 (segment (start 146.8725 118.3) (end 146.8725 119.535388) (width 0.25) (layer F.Cu) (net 51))
 (segment (start 142.722489 133.176569) (end 144.005879 134.459959) (width 0.25) (layer F.Cu) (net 50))
 (segment (start 142.722489 124.321809) (end 142.722489 133.176569) (width 0.25) (layer F.Cu) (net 50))
 (segment (start 147.5075 119.536798) (end 142.722489 124.321809) (width 0.25) (layer F.Cu) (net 50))
 (segment (start 147.5075 118.3) (end 147.5075 119.536798) (width 0.25) (layer F.Cu) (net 50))
 (segment (start 143.172499 131.086579) (end 146.545879 134.459959) (width 0.25) (layer F.Cu) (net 49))
 (segment (start 143.172499 124.508209) (end 143.172499 131.086579) (width 0.25) (layer F.Cu) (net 49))
 (segment (start 148.1425 119.538208) (end 143.172499 124.508209) (width 0.25) (layer F.Cu) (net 49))
 (segment (start 148.1425 118.3) (end 148.1425 119.538208) (width 0.25) (layer F.Cu) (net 49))
 (segment (start 148.7775 117.549998) (end 148.602501 117.374999) (width 0.25) (layer F.Cu) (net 21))
 (segment (start 148.7775 118.3) (end 148.7775 117.549998) (width 0.25) (layer F.Cu) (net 21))
 (segment (start 135.653879 117.374999) (end 128.765879 110.486999) (width 0.25) (layer F.Cu) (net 21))
 (segment (start 148.602501 117.374999) (end 135.653879 117.374999) (width 0.25) (layer F.Cu) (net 21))
 (segment (start 149.4125 117.548588) (end 148.788901 116.924989) (width 0.25) (layer F.Cu) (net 22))
 (segment (start 149.4125 118.3) (end 149.4125 117.548588) (width 0.25) (layer F.Cu) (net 22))
 (segment (start 137.743869 116.924989) (end 131.305879 110.486999) (width 0.25) (layer F.Cu) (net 22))
 (segment (start 148.788901 116.924989) (end 137.743869 116.924989) (width 0.25) (layer F.Cu) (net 22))
 (segment (start 150.0475 117.547178) (end 148.975301 116.474979) (width 0.25) (layer F.Cu) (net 23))
 (segment (start 150.0475 118.3) (end 150.0475 117.547178) (width 0.25) (layer F.Cu) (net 23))
 (segment (start 139.833859 116.474979) (end 133.845879 110.486999) (width 0.25) (layer F.Cu) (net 23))
 (segment (start 148.975301 116.474979) (end 139.833859 116.474979) (width 0.25) (layer F.Cu) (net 23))
 (segment (start 150.6825 117.45) (end 149.257469 116.024969) (width 0.25) (layer F.Cu) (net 24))
 (segment (start 150.6825 118.3) (end 150.6825 117.45) (width 0.25) (layer F.Cu) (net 24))
 (segment (start 141.923849 116.024969) (end 136.385879 110.486999) (width 0.25) (layer F.Cu) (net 24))
 (segment (start 149.257469 116.024969) (end 141.923849 116.024969) (width 0.25) (layer F.Cu) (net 24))
 (segment (start 151.3175 117.44859) (end 149.443869 115.574959) (width 0.25) (layer F.Cu) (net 25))
 (segment (start 151.3175 118.3) (end 151.3175 117.44859) (width 0.25) (layer F.Cu) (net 25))
 (segment (start 144.013839 115.574959) (end 138.925879 110.486999) (width 0.25) (layer F.Cu) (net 25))
 (segment (start 149.443869 115.574959) (end 144.013839 115.574959) (width 0.25) (layer F.Cu) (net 25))
 (segment (start 151.9525 118.3) (end 151.9525 117.44718) (width 0.25) (layer F.Cu) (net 26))
 (segment (start 151.9525 117.44718) (end 149.630269 115.124949) (width 0.25) (layer F.Cu) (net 26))
 (segment (start 146.103829 115.124949) (end 141.465879 110.486999) (width 0.25) (layer F.Cu) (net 26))
 (segment (start 149.630269 115.124949) (end 146.103829 115.124949) (width 0.25) (layer F.Cu) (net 26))
 (segment (start 152.5875 117.44577) (end 149.816669 114.674939) (width 0.25) (layer F.Cu) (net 27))
 (segment (start 152.5875 118.3) (end 152.5875 117.44577) (width 0.25) (layer F.Cu) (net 27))
 (segment (start 148.193819 114.674939) (end 144.005879 110.486999) (width 0.25) (layer F.Cu) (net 27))
 (segment (start 149.816669 114.674939) (end 148.193819 114.674939) (width 0.25) (layer F.Cu) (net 27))
 (segment (start 153.2225 117.16362) (end 153.2225 118.3) (width 0.25) (layer F.Cu) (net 28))
 (segment (start 146.545879 110.486999) (end 153.2225 117.16362) (width 0.25) (layer F.Cu) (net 28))
 (segment (start 153.8575 115.25862) (end 153.8575 118.3) (width 0.25) (layer F.Cu) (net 29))
 (segment (start 149.085879 110.486999) (end 153.8575 115.25862) (width 0.25) (layer F.Cu) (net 29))
 (segment (start 154.4925 113.35362) (end 154.4925 118.3) (width 0.25) (layer F.Cu) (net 30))
 (segment (start 151.625879 110.486999) (end 154.4925 113.35362) (width 0.25) (layer F.Cu) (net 30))
 (segment (start 155.1275 111.44862) (end 155.1275 118.3) (width 0.25) (layer F.Cu) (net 31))
 (segment (start 154.165879 110.486999) (end 155.1275 111.44862) (width 0.25) (layer F.Cu) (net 31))
 (segment (start 155.7625 111.430378) (end 155.7625 118.3) (width 0.25) (layer F.Cu) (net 32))
 (segment (start 156.705879 110.486999) (end 155.7625 111.430378) (width 0.25) (layer F.Cu) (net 32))
 (segment (start 156.3975 113.335378) (end 156.3975 118.3) (width 0.25) (layer F.Cu) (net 33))
 (segment (start 159.245879 110.486999) (end 156.3975 113.335378) (width 0.25) (layer F.Cu) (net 33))
 (segment (start 157.0325 115.240378) (end 157.0325 118.3) (width 0.25) (layer F.Cu) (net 34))
 (segment (start 161.785879 110.486999) (end 157.0325 115.240378) (width 0.25) (layer F.Cu) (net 34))
 (segment (start 157.6675 117.145378) (end 157.6675 118.3) (width 0.25) (layer F.Cu) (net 35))
 (segment (start 164.325879 110.486999) (end 157.6675 117.145378) (width 0.25) (layer F.Cu) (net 35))
 (segment (start 159.052878 118.3) (end 166.865879 110.486999) (width 0.25) (layer F.Cu) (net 36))
 (segment (start 158.3025 118.3) (end 159.052878 118.3) (width 0.25) (layer F.Cu) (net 36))
 (segment (start 161.40592 129) (end 166.865879 134.459959) (width 0.25) (layer F.Cu) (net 41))
 (segment (start 148.692498 129) (end 161.40592 129) (width 0.25) (layer F.Cu) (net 41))
 (segment (start 148.1425 128.450002) (end 148.692498 129) (width 0.25) (layer F.Cu) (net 41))
 (segment (start 148.1425 127.7) (end 148.1425 128.450002) (width 0.25) (layer F.Cu) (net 41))
 (segment (start 147.5075 127.7) (end 147.5075 128.5075) (width 0.25) (layer F.Cu) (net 42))
 (segment (start 159.31593 129.45001) (end 164.325879 134.459959) (width 0.25) (layer F.Cu) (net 42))
 (segment (start 148.45001 129.45001) (end 159.31593 129.45001) (width 0.25) (layer F.Cu) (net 42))
 (segment (start 147.5075 128.5075) (end 148.45001 129.45001) (width 0.25) (layer F.Cu) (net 42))
 (segment (start 146.8725 128.50891) (end 148.26361 129.90002) (width 0.25) (layer F.Cu) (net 43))
 (segment (start 146.8725 127.7) (end 146.8725 128.50891) (width 0.25) (layer F.Cu) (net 43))
 (segment (start 157.22594 129.90002) (end 161.785879 134.459959) (width 0.25) (layer F.Cu) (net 43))
 (segment (start 148.26361 129.90002) (end 157.22594 129.90002) (width 0.25) (layer F.Cu) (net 43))
 (segment (start 146.422491 128.695311) (end 148.07721 130.35003) (width 0.25) (layer F.Cu) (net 44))
 (segment (start 146.42249 128.634992) (end 146.422491 128.695311) (width 0.25) (layer F.Cu) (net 44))
 (segment (start 146.2375 128.450002) (end 146.42249 128.634992) (width 0.25) (layer F.Cu) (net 44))
 (segment (start 146.2375 127.7) (end 146.2375 128.450002) (width 0.25) (layer F.Cu) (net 44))
 (segment (start 155.13595 130.35003) (end 159.245879 134.459959) (width 0.25) (layer F.Cu) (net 44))
 (segment (start 148.07721 130.35003) (end 155.13595 130.35003) (width 0.25) (layer F.Cu) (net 44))
 (segment (start 145.6025 128.51173) (end 147.89081 130.80004) (width 0.25) (layer F.Cu) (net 45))
 (segment (start 145.6025 127.7) (end 145.6025 128.51173) (width 0.25) (layer F.Cu) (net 45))
 (segment (start 153.04596 130.80004) (end 156.705879 134.459959) (width 0.25) (layer F.Cu) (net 45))
 (segment (start 147.89081 130.80004) (end 153.04596 130.80004) (width 0.25) (layer F.Cu) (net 45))
 (segment (start 144.9675 128.55) (end 147 130.5825) (width 0.25) (layer F.Cu) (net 46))
 (segment (start 144.9675 127.7) (end 144.9675 128.55) (width 0.25) (layer F.Cu) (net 46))
 (segment (start 147.03686 130.5825) (end 147.70441 131.25005) (width 0.25) (layer F.Cu) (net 46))
 (segment (start 147 130.5825) (end 147.03686 130.5825) (width 0.25) (layer F.Cu) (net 46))
 (segment (start 150.95597 131.25005) (end 154.165879 134.459959) (width 0.25) (layer F.Cu) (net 46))
 (segment (start 147.70441 131.25005) (end 150.95597 131.25005) (width 0.25) (layer F.Cu) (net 46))
 (segment (start 144.3325 127.7) (end 144.3325 128.5825) (width 0.25) (layer F.Cu) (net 47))
 (segment (start 144.3325 128.5825) (end 147.450059 131.700059) (width 0.25) (layer F.Cu) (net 47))
 (segment (start 148.865979 131.700059) (end 151.625879 134.459959) (width 0.25) (layer F.Cu) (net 47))
 (segment (start 147.450059 131.700059) (end 148.865979 131.700059) (width 0.25) (layer F.Cu) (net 47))
 (segment (start 143.88249 128.73499) (end 143.882491 128.768901) (width 0.25) (layer F.Cu) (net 48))
 (segment (start 143.6975 128.55) (end 143.88249 128.73499) (width 0.25) (layer F.Cu) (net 48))
 (segment (start 143.6975 127.7) (end 143.6975 128.55) (width 0.25) (layer F.Cu) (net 48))
 (segment (start 149.085879 133.972289) (end 149.085879 134.459959) (width 0.25) (layer F.Cu) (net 48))
 (segment (start 143.882491 128.768901) (end 149.085879 133.972289) (width 0.25) (layer F.Cu) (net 48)))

